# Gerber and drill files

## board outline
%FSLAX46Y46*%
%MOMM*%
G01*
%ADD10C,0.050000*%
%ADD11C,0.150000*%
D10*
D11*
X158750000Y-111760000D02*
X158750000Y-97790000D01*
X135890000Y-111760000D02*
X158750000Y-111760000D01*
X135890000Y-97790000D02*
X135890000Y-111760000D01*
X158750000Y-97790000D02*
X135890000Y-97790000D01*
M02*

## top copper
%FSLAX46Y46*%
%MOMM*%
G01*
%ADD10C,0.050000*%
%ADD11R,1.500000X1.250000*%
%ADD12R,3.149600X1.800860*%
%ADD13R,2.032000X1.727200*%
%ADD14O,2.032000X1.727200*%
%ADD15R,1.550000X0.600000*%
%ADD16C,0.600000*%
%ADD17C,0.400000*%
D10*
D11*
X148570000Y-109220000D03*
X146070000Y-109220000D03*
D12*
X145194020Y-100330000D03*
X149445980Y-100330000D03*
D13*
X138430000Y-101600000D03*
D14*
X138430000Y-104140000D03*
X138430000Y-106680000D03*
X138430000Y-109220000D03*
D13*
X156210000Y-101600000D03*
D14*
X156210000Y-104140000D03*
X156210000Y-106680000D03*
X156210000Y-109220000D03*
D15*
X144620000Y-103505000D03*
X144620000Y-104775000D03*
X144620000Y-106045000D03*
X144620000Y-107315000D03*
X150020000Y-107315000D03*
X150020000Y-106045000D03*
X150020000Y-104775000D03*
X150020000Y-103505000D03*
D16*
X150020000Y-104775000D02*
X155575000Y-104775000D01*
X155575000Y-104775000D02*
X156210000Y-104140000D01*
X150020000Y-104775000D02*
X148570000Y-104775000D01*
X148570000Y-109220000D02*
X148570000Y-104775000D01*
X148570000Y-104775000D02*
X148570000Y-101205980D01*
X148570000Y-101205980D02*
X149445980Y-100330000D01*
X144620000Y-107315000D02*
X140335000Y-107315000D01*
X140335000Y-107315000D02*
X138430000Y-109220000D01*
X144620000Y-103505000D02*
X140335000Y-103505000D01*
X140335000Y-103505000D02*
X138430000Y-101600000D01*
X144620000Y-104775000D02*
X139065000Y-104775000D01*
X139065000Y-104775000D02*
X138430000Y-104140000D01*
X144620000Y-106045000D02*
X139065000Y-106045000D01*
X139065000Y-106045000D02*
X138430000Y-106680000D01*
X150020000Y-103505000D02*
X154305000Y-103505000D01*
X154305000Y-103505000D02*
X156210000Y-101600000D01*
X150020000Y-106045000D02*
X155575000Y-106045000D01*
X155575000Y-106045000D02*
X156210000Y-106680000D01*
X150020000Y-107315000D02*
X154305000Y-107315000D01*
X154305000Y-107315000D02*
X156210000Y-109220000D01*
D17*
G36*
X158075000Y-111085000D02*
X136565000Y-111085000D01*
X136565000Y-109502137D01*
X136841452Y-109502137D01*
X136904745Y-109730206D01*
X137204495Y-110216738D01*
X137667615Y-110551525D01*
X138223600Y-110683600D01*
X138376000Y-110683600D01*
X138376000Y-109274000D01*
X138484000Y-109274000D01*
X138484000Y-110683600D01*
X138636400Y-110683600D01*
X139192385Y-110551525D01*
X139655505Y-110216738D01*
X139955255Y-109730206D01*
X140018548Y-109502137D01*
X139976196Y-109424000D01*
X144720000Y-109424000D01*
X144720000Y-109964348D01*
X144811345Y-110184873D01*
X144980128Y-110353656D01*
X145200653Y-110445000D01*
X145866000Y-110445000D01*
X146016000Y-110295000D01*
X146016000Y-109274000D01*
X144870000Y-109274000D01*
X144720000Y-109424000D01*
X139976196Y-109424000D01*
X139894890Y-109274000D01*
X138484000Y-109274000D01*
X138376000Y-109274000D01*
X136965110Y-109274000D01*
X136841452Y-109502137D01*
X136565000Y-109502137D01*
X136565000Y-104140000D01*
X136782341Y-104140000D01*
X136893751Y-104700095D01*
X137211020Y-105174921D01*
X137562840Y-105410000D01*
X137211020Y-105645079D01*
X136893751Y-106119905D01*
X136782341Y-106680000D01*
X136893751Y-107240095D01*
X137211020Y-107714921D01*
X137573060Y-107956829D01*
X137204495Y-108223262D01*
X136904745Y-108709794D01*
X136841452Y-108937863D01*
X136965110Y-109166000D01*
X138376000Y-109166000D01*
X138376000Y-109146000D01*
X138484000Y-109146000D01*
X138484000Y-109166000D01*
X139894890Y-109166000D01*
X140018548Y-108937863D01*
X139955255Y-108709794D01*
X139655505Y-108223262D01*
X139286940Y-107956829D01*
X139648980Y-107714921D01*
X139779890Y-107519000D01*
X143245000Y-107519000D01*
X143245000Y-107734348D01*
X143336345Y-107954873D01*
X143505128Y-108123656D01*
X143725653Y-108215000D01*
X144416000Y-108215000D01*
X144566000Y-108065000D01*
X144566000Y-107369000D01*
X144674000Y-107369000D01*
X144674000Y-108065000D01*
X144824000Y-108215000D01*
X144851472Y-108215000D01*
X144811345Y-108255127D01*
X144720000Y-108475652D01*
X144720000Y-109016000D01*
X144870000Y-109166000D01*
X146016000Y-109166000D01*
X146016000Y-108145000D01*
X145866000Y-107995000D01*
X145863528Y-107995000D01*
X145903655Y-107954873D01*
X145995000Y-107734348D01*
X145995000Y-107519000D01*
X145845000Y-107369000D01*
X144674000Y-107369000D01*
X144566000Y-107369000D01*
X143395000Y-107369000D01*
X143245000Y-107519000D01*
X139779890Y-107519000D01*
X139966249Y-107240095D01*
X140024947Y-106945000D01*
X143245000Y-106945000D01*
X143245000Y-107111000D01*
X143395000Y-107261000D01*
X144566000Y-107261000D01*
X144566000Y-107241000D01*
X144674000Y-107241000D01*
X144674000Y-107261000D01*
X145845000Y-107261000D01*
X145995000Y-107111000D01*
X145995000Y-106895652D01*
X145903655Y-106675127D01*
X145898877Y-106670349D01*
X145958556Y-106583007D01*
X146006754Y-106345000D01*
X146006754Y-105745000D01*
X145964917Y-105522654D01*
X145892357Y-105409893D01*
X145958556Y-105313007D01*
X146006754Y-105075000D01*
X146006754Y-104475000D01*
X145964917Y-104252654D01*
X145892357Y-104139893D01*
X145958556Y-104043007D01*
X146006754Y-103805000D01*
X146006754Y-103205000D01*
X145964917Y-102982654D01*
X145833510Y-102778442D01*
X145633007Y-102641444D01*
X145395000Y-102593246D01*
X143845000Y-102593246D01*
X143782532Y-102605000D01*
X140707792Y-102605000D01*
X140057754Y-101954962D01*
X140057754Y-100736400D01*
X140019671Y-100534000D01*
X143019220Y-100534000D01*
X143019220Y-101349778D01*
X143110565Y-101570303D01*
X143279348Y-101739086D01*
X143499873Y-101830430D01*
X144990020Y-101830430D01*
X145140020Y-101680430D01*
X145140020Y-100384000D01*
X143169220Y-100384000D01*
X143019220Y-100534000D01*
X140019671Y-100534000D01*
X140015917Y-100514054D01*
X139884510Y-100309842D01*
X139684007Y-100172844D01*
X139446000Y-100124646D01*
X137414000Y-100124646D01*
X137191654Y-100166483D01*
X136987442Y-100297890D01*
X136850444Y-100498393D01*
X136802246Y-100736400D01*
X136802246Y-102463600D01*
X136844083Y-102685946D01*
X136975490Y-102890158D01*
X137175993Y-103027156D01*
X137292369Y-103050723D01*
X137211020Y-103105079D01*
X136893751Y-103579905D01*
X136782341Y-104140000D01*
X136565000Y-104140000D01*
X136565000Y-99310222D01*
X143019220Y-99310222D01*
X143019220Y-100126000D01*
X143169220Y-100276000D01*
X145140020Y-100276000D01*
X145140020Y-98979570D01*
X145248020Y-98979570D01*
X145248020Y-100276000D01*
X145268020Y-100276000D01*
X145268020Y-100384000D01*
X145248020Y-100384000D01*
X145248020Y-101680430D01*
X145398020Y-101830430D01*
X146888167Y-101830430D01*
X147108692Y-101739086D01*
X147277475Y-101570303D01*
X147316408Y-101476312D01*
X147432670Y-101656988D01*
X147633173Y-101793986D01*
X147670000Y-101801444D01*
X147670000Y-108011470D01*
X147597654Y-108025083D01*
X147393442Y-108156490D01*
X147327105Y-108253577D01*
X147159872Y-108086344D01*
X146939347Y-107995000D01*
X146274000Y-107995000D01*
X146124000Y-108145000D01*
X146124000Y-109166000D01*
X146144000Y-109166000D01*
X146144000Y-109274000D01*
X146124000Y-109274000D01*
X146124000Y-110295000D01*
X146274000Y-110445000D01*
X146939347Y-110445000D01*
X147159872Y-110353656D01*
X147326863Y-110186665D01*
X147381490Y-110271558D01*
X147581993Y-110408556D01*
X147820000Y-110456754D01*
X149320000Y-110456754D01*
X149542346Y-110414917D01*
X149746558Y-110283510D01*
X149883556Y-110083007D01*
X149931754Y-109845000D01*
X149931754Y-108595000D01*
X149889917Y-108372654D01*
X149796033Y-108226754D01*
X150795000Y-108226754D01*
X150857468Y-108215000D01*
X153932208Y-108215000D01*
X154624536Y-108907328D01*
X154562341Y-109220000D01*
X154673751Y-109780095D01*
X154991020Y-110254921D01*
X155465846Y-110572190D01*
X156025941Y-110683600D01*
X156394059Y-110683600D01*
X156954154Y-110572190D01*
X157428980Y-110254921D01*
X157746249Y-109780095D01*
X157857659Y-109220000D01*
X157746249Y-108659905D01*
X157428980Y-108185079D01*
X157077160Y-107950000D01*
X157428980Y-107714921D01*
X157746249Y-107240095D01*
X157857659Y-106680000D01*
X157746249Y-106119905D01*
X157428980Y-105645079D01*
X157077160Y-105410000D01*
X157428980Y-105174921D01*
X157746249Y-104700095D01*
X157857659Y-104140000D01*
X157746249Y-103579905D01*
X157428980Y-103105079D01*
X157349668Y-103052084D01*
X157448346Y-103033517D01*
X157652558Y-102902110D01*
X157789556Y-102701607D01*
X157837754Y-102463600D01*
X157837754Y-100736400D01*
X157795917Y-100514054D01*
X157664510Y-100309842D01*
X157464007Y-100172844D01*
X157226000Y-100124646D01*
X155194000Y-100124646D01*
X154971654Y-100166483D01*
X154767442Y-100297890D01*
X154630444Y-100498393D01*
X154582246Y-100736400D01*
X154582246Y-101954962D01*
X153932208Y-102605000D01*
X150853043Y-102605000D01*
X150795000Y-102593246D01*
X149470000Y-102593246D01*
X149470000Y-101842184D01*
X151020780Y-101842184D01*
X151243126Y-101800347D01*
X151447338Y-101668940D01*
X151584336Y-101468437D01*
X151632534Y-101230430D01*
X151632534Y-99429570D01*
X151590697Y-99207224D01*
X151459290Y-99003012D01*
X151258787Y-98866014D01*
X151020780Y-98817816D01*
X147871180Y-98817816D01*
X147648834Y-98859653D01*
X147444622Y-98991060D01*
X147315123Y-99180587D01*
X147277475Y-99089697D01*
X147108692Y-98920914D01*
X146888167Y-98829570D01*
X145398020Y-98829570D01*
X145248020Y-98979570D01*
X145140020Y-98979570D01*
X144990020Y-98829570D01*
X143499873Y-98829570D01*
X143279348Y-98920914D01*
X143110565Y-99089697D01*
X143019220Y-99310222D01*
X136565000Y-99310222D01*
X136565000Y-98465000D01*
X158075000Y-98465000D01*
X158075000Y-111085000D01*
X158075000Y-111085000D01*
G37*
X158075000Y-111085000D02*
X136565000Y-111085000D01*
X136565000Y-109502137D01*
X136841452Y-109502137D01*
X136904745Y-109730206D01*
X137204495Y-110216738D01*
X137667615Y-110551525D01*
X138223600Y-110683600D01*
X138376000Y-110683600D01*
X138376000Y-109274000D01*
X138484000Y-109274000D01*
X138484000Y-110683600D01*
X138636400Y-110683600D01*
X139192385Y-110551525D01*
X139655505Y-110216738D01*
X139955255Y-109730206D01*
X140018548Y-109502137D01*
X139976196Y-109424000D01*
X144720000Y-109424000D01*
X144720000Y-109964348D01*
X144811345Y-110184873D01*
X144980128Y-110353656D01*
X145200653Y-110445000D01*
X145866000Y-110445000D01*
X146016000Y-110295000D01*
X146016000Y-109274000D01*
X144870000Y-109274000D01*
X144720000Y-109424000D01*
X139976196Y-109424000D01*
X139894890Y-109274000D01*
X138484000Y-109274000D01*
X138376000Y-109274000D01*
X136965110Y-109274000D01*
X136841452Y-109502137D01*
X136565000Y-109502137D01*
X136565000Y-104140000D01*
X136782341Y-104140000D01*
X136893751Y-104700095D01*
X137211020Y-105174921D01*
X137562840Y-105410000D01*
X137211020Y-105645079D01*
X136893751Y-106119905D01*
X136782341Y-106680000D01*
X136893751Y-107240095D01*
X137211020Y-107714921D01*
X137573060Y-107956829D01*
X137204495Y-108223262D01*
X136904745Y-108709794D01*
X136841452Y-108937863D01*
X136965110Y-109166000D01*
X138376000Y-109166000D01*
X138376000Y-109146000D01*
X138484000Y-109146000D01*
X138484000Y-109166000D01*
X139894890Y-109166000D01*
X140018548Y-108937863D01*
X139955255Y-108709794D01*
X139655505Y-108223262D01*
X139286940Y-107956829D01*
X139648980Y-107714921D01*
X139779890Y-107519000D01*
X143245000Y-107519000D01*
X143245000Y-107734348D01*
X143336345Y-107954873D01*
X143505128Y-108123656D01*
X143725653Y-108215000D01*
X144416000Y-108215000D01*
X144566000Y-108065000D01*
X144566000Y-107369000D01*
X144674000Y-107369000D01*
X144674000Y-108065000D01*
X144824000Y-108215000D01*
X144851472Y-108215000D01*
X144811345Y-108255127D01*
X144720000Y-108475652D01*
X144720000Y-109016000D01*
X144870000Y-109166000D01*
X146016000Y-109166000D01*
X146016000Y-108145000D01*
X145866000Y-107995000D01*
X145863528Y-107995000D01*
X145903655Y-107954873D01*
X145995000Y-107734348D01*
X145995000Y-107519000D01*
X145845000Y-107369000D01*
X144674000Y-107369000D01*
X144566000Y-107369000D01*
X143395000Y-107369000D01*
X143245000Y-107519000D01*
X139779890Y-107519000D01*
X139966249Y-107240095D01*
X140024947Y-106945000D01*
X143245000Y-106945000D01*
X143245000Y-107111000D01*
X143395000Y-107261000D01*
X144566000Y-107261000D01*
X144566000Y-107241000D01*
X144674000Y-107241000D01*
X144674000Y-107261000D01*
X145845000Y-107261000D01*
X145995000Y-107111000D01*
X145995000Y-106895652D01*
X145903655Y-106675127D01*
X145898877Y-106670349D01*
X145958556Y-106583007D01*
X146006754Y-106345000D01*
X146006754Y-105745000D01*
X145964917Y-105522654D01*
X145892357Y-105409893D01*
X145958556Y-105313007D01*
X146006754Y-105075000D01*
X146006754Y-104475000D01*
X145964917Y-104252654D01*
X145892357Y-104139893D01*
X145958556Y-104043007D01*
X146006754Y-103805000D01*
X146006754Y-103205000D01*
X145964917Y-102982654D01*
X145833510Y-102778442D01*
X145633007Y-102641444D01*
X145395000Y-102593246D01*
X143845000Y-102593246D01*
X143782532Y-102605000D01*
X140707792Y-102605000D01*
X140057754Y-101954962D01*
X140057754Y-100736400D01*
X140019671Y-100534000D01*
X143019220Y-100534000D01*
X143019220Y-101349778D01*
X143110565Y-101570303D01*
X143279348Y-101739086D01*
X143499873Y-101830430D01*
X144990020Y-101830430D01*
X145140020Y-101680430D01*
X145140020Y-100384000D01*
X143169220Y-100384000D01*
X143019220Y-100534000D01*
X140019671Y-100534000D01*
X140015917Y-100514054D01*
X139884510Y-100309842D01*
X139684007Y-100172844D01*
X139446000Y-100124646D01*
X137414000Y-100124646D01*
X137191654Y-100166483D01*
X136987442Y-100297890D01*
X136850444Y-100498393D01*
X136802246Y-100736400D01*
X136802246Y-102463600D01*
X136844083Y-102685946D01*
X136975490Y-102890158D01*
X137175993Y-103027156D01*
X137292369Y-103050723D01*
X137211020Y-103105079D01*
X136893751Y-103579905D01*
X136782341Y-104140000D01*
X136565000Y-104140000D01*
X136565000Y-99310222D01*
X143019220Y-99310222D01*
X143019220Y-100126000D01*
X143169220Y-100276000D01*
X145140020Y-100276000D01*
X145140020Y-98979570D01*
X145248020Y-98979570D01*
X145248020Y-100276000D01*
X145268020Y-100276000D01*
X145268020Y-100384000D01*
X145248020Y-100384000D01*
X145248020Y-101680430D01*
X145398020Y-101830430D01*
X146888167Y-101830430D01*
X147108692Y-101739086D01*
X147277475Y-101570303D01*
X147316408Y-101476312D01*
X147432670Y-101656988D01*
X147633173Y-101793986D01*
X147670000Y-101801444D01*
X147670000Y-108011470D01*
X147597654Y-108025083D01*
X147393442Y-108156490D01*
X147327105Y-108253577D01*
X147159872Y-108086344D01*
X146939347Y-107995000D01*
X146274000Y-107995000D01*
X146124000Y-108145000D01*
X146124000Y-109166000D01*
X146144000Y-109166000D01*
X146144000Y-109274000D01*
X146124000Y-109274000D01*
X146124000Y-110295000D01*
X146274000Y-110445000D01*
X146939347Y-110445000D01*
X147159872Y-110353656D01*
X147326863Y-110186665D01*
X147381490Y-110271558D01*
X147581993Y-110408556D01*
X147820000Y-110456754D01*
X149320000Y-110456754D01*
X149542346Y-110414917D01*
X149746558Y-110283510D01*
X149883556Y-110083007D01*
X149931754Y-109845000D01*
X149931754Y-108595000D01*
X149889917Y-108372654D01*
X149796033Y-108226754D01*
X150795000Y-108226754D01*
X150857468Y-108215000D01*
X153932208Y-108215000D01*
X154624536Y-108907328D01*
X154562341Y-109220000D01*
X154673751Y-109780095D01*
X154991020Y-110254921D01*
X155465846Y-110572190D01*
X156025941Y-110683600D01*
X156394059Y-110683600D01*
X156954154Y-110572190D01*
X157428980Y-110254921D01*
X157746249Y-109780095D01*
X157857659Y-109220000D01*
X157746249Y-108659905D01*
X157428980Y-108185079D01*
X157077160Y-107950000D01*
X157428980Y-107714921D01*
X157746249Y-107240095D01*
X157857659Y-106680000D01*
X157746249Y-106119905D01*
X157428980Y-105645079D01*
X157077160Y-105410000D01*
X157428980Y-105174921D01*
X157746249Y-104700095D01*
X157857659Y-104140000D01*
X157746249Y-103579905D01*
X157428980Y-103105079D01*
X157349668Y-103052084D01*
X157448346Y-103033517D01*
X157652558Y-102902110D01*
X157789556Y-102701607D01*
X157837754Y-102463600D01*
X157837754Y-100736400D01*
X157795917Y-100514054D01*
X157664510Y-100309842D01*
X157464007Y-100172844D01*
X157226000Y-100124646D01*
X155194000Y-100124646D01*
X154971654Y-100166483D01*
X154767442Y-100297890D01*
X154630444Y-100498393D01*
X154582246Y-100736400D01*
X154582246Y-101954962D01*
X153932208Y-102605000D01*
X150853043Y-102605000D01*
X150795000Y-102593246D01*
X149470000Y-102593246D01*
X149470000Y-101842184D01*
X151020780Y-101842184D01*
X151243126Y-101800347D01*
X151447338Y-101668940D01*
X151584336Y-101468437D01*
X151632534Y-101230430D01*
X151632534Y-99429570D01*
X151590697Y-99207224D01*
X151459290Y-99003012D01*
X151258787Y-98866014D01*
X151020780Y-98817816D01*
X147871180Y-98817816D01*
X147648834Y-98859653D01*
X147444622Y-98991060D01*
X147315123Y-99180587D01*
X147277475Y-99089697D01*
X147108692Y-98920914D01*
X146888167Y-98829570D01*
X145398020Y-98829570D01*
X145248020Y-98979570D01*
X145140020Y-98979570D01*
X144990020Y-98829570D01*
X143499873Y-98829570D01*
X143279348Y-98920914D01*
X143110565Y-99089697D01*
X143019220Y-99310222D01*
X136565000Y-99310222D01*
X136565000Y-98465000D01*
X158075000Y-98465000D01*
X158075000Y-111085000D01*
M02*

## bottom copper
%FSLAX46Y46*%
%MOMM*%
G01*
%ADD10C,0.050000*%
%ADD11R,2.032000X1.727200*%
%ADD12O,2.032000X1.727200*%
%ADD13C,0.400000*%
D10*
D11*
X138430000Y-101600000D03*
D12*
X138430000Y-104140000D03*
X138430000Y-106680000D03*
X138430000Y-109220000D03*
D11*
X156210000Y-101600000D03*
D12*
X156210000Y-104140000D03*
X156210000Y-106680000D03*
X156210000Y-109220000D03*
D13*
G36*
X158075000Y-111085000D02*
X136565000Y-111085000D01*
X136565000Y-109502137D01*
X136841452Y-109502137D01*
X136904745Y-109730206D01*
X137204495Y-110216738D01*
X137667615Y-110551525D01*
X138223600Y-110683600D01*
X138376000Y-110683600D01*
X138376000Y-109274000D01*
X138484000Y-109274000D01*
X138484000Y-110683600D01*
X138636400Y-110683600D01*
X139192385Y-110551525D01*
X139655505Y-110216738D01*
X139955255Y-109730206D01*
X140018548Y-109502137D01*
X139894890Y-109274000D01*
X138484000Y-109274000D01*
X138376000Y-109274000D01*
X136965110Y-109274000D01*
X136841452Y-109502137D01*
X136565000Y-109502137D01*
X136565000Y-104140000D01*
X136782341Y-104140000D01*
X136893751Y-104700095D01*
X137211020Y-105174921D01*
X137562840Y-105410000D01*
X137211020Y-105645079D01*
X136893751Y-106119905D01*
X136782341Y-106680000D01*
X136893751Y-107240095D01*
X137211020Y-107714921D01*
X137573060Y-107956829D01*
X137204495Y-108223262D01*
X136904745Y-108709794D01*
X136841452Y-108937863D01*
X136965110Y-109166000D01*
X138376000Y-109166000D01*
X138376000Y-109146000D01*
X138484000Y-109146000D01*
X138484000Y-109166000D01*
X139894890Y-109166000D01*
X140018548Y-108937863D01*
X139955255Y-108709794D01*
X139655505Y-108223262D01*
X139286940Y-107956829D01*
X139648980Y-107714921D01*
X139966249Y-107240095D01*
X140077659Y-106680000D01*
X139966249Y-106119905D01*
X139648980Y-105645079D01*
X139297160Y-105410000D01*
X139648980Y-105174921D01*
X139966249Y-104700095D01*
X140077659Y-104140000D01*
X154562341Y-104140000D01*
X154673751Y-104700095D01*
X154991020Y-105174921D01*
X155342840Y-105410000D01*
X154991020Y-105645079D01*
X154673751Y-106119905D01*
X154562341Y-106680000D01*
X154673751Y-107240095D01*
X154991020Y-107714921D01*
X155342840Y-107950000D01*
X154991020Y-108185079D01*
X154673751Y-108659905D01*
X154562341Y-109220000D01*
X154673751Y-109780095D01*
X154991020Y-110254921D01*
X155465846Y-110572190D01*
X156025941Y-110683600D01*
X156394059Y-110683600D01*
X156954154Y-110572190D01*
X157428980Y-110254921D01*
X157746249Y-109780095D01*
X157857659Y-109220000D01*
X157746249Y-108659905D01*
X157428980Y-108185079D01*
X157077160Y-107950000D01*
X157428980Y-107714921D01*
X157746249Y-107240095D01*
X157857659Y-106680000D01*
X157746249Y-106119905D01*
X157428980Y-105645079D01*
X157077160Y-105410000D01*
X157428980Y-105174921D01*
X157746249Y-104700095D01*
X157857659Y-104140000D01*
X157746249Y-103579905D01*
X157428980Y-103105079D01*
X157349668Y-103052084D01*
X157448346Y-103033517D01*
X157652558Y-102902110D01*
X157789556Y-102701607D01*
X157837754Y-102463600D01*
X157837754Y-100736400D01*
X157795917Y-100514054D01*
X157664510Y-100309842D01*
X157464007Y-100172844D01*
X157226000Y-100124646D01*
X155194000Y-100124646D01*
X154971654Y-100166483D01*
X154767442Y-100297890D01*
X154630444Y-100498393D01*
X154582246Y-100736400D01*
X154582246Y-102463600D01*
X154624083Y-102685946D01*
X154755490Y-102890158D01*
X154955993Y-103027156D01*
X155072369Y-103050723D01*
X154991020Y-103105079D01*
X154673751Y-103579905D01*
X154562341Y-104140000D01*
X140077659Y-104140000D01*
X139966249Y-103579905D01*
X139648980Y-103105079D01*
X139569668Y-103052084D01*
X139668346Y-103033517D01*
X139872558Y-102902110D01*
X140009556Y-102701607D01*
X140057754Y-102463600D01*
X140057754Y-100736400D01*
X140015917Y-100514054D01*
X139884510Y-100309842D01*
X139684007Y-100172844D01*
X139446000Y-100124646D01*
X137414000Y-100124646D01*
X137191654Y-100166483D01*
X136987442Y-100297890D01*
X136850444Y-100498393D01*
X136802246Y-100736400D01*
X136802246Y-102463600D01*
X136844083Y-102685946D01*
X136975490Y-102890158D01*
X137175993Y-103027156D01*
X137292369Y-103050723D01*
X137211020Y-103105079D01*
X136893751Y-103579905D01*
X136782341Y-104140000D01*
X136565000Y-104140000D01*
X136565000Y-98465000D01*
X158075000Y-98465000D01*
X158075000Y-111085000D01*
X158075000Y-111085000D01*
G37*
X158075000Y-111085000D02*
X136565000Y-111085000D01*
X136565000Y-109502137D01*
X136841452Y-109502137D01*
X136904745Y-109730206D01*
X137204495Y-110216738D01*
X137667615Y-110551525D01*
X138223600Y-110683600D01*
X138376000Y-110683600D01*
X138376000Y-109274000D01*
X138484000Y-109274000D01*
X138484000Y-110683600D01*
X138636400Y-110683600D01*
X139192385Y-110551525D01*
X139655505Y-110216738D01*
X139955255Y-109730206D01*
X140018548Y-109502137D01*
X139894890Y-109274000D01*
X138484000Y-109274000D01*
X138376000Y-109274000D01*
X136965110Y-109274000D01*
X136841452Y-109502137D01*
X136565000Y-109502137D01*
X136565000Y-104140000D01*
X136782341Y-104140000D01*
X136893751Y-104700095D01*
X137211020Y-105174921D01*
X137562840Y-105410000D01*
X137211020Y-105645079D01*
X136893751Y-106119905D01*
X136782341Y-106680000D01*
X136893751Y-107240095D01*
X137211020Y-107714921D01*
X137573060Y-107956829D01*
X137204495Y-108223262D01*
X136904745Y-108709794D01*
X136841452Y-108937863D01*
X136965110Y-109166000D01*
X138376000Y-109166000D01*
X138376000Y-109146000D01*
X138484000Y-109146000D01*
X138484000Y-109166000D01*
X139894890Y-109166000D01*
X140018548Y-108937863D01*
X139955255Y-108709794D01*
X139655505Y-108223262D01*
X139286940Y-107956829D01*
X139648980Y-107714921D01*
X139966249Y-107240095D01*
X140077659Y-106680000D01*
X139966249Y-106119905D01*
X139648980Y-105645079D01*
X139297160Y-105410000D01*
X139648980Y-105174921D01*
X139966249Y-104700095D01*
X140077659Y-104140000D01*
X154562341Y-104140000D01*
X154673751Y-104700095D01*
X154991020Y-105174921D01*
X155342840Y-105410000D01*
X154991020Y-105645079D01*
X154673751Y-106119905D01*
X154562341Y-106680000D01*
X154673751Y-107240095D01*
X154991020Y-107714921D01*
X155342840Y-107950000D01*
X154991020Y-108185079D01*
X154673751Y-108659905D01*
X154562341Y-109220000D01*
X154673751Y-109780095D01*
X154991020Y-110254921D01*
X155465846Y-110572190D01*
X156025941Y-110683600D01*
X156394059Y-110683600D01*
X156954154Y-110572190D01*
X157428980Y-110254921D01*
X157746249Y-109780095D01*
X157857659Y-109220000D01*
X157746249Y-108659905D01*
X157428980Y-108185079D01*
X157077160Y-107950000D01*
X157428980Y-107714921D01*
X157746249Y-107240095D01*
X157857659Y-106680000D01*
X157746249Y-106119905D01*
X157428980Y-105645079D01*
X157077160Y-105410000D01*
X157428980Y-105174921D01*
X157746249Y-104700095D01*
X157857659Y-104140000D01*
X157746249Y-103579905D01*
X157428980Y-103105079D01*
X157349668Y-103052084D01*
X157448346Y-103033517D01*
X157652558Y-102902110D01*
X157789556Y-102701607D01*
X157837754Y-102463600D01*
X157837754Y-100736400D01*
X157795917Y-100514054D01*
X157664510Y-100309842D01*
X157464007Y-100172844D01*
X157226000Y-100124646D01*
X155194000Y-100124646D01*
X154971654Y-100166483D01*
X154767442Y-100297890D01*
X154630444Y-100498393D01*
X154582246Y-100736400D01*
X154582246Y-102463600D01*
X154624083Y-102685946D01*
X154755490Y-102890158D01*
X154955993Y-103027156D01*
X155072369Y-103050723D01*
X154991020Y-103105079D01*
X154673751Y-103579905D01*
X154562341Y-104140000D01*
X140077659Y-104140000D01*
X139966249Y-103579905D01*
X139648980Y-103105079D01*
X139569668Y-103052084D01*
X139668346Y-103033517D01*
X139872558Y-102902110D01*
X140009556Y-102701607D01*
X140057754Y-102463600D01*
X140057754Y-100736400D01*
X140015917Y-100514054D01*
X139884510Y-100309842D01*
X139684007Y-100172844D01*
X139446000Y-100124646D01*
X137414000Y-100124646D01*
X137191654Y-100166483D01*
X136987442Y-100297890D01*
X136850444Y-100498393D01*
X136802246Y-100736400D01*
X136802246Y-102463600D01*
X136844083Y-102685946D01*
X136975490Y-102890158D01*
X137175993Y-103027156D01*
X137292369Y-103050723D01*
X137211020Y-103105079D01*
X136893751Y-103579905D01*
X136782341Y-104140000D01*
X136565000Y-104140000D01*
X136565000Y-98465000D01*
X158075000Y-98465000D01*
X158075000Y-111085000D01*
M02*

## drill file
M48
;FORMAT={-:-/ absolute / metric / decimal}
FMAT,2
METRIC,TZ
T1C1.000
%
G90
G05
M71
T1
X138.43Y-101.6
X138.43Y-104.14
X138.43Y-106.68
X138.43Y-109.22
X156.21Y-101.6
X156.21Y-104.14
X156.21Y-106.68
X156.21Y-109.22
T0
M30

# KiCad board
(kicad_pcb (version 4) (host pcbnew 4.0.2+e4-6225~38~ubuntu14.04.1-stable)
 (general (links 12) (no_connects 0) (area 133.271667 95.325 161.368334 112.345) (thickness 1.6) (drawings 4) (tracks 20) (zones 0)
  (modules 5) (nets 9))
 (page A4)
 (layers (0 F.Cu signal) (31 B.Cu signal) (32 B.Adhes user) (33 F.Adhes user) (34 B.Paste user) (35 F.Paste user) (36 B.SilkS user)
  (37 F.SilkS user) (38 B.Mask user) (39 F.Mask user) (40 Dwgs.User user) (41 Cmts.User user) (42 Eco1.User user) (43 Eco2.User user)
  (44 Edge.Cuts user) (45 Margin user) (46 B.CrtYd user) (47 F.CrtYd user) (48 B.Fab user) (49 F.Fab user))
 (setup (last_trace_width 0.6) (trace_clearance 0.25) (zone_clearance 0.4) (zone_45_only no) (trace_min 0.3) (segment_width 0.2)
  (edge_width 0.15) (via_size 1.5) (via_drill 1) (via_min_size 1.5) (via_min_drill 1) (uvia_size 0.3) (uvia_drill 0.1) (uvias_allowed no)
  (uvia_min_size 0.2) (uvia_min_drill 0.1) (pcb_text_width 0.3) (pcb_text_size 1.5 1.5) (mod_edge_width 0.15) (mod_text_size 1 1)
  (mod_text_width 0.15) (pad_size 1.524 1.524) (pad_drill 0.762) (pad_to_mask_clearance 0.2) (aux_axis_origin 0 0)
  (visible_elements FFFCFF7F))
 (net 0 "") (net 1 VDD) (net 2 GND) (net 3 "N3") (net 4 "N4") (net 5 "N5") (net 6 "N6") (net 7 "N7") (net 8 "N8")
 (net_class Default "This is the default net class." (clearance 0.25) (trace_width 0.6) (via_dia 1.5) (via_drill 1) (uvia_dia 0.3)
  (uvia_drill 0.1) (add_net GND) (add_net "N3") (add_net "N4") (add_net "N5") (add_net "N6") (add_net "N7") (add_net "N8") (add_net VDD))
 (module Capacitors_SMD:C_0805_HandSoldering (layer F.Cu) (at 147.32 109.22 180)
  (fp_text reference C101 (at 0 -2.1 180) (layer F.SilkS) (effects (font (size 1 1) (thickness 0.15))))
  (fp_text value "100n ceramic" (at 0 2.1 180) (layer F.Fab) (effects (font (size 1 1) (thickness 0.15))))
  (pad 1 smd rect (at -1.25 0 180) (size 1.5 1.25) (layers F.Cu F.Paste F.Mask) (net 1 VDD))
  (pad 2 smd rect (at 1.25 0 180) (size 1.5 1.25) (layers F.Cu F.Paste F.Mask) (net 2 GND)))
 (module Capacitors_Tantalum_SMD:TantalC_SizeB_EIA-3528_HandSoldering (layer F.Cu) (at 147.32 100.33 180)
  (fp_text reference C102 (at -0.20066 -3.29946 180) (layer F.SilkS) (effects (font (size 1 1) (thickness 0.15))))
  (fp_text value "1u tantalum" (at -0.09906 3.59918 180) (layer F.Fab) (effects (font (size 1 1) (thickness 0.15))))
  (pad 2 smd rect (at 2.12598 0 180) (size 3.1496 1.80086) (layers F.Cu F.Paste F.Mask) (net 2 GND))
  (pad 1 smd rect (at -2.12598 0 180) (size 3.1496 1.80086) (layers F.Cu F.Paste F.Mask) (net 1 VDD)))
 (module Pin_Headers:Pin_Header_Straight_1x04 (layer F.Cu) (at 138.43 101.6)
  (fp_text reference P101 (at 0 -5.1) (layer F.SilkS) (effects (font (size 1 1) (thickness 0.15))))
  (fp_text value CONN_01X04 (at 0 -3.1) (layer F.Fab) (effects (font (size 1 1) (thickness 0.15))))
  (pad 1 thru_hole rect (at 0 0) (size 2.032 1.7272) (drill 1.016) (layers *.Cu *.Mask F.SilkS) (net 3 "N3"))
  (pad 2 thru_hole oval (at 0 2.54) (size 2.032 1.7272) (drill 1.016) (layers *.Cu *.Mask F.SilkS) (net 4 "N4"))
  (pad 3 thru_hole oval (at 0 5.08) (size 2.032 1.7272) (drill 1.016) (layers *.Cu *.Mask F.SilkS) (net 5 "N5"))
  (pad 4 thru_hole oval (at 0 7.62) (size 2.032 1.7272) (drill 1.016) (layers *.Cu *.Mask F.SilkS) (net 2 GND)))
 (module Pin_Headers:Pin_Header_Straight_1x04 (layer F.Cu) (at 156.21 101.6)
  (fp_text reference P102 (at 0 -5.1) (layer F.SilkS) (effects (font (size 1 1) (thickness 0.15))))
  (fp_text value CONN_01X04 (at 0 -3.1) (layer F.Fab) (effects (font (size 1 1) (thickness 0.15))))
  (pad 1 thru_hole rect (at 0 0) (size 2.032 1.7272) (drill 1.016) (layers *.Cu *.Mask F.SilkS) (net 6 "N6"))
  (pad 2 thru_hole oval (at 0 2.54) (size 2.032 1.7272) (drill 1.016) (layers *.Cu *.Mask F.SilkS) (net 1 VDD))
  (pad 3 thru_hole oval (at 0 5.08) (size 2.032 1.7272) (drill 1.016) (layers *.Cu *.Mask F.SilkS) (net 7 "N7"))
  (pad 4 thru_hole oval (at 0 7.62) (size 2.032 1.7272) (drill 1.016) (layers *.Cu *.Mask F.SilkS) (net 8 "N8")))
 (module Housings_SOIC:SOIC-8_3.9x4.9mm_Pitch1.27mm (layer F.Cu) (at 147.32 105.41)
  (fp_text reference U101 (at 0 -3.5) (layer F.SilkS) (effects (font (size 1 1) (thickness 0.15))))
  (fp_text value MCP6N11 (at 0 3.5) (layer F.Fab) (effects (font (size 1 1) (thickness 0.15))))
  (pad 1 smd rect (at -2.7 -1.905) (size 1.55 0.6) (layers F.Cu F.Paste F.Mask) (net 3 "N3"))
  (pad 2 smd rect (at -2.7 -0.635) (size 1.55 0.6) (layers F.Cu F.Paste F.Mask) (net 4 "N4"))
  (pad 3 smd rect (at -2.7 0.635) (size 1.55 0.6) (layers F.Cu F.Paste F.Mask) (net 5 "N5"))
  (pad 4 smd rect (at -2.7 1.905) (size 1.55 0.6) (layers F.Cu F.Paste F.Mask) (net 2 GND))
  (pad 5 smd rect (at 2.7 1.905) (size 1.55 0.6) (layers F.Cu F.Paste F.Mask) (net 8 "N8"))
  (pad 6 smd rect (at 2.7 0.635) (size 1.55 0.6) (layers F.Cu F.Paste F.Mask) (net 7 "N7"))
  (pad 7 smd rect (at 2.7 -0.635) (size 1.55 0.6) (layers F.Cu F.Paste F.Mask) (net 1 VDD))
  (pad 8 smd rect (at 2.7 -1.905) (size 1.55 0.6) (layers F.Cu F.Paste F.Mask) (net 6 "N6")))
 (gr_line (start 158.75 111.76) (end 158.75 97.79) (angle 90) (layer Edge.Cuts) (width 0.15))
 (gr_line (start 135.89 111.76) (end 158.75 111.76) (angle 90) (layer Edge.Cuts) (width 0.15))
 (gr_line (start 135.89 97.79) (end 135.89 111.76) (angle 90) (layer Edge.Cuts) (width 0.15))
 (gr_line (start 158.75 97.79) (end 135.89 97.79) (angle 90) (layer Edge.Cuts) (width 0.15))
 (segment (start 150.02 104.775) (end 155.575 104.775) (width 0.6) (layer F.Cu) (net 1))
 (segment (start 155.575 104.775) (end 156.21 104.14) (width 0.6) (layer F.Cu) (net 1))
 (segment (start 150.02 104.775) (end 148.57 104.775) (width 0.6) (layer F.Cu) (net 1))
 (segment (start 148.57 109.22) (end 148.57 104.775) (width 0.6) (layer F.Cu) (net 1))
 (segment (start 148.57 104.775) (end 148.57 101.20598) (width 0.6) (layer F.Cu) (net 1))
 (segment (start 148.57 101.20598) (end 149.44598 100.33) (width 0.6) (layer F.Cu) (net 1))
 (segment (start 144.62 107.315) (end 140.335 107.315) (width 0.6) (layer F.Cu) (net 2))
 (segment (start 140.335 107.315) (end 138.43 109.22) (width 0.6) (layer F.Cu) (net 2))
 (segment (start 144.62 103.505) (end 140.335 103.505) (width 0.6) (layer F.Cu) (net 3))
 (segment (start 140.335 103.505) (end 138.43 101.6) (width 0.6) (layer F.Cu) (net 3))
 (segment (start 144.62 104.775) (end 139.065 104.775) (width 0.6) (layer F.Cu) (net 4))
 (segment (start 139.065 104.775) (end 138.43 104.14) (width 0.6) (layer F.Cu) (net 4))
 (segment (start 144.62 106.045) (end 139.065 106.045) (width 0.6) (layer F.Cu) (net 5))
 (segment (start 139.065 106.045) (end 138.43 106.68) (width 0.6) (layer F.Cu) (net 5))
 (segment (start 150.02 103.505) (end 154.305 103.505) (width 0.6) (layer F.Cu) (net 6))
 (segment (start 154.305 103.505) (end 156.21 101.6) (width 0.6) (layer F.Cu) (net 6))
 (segment (start 150.02 106.045) (end 155.575 106.045) (width 0.6) (layer F.Cu) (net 7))
 (segment (start 155.575 106.045) (end 156.21 106.68) (width 0.6) (layer F.Cu) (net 7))
 (segment (start 150.02 107.315) (end 154.305 107.315) (width 0.6) (layer F.Cu) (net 8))
 (segment (start 154.305 107.315) (end 156.21 109.22) (width 0.6) (layer F.Cu) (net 8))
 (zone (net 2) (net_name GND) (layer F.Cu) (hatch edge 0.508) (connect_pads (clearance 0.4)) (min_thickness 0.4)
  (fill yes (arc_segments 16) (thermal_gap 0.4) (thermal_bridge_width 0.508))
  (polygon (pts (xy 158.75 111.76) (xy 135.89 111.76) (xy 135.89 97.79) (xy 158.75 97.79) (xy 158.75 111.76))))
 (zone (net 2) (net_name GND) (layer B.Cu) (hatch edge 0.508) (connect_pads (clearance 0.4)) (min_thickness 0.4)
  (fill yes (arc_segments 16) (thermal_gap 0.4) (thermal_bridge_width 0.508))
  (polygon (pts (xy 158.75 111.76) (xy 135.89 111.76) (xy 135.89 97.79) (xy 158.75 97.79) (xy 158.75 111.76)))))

